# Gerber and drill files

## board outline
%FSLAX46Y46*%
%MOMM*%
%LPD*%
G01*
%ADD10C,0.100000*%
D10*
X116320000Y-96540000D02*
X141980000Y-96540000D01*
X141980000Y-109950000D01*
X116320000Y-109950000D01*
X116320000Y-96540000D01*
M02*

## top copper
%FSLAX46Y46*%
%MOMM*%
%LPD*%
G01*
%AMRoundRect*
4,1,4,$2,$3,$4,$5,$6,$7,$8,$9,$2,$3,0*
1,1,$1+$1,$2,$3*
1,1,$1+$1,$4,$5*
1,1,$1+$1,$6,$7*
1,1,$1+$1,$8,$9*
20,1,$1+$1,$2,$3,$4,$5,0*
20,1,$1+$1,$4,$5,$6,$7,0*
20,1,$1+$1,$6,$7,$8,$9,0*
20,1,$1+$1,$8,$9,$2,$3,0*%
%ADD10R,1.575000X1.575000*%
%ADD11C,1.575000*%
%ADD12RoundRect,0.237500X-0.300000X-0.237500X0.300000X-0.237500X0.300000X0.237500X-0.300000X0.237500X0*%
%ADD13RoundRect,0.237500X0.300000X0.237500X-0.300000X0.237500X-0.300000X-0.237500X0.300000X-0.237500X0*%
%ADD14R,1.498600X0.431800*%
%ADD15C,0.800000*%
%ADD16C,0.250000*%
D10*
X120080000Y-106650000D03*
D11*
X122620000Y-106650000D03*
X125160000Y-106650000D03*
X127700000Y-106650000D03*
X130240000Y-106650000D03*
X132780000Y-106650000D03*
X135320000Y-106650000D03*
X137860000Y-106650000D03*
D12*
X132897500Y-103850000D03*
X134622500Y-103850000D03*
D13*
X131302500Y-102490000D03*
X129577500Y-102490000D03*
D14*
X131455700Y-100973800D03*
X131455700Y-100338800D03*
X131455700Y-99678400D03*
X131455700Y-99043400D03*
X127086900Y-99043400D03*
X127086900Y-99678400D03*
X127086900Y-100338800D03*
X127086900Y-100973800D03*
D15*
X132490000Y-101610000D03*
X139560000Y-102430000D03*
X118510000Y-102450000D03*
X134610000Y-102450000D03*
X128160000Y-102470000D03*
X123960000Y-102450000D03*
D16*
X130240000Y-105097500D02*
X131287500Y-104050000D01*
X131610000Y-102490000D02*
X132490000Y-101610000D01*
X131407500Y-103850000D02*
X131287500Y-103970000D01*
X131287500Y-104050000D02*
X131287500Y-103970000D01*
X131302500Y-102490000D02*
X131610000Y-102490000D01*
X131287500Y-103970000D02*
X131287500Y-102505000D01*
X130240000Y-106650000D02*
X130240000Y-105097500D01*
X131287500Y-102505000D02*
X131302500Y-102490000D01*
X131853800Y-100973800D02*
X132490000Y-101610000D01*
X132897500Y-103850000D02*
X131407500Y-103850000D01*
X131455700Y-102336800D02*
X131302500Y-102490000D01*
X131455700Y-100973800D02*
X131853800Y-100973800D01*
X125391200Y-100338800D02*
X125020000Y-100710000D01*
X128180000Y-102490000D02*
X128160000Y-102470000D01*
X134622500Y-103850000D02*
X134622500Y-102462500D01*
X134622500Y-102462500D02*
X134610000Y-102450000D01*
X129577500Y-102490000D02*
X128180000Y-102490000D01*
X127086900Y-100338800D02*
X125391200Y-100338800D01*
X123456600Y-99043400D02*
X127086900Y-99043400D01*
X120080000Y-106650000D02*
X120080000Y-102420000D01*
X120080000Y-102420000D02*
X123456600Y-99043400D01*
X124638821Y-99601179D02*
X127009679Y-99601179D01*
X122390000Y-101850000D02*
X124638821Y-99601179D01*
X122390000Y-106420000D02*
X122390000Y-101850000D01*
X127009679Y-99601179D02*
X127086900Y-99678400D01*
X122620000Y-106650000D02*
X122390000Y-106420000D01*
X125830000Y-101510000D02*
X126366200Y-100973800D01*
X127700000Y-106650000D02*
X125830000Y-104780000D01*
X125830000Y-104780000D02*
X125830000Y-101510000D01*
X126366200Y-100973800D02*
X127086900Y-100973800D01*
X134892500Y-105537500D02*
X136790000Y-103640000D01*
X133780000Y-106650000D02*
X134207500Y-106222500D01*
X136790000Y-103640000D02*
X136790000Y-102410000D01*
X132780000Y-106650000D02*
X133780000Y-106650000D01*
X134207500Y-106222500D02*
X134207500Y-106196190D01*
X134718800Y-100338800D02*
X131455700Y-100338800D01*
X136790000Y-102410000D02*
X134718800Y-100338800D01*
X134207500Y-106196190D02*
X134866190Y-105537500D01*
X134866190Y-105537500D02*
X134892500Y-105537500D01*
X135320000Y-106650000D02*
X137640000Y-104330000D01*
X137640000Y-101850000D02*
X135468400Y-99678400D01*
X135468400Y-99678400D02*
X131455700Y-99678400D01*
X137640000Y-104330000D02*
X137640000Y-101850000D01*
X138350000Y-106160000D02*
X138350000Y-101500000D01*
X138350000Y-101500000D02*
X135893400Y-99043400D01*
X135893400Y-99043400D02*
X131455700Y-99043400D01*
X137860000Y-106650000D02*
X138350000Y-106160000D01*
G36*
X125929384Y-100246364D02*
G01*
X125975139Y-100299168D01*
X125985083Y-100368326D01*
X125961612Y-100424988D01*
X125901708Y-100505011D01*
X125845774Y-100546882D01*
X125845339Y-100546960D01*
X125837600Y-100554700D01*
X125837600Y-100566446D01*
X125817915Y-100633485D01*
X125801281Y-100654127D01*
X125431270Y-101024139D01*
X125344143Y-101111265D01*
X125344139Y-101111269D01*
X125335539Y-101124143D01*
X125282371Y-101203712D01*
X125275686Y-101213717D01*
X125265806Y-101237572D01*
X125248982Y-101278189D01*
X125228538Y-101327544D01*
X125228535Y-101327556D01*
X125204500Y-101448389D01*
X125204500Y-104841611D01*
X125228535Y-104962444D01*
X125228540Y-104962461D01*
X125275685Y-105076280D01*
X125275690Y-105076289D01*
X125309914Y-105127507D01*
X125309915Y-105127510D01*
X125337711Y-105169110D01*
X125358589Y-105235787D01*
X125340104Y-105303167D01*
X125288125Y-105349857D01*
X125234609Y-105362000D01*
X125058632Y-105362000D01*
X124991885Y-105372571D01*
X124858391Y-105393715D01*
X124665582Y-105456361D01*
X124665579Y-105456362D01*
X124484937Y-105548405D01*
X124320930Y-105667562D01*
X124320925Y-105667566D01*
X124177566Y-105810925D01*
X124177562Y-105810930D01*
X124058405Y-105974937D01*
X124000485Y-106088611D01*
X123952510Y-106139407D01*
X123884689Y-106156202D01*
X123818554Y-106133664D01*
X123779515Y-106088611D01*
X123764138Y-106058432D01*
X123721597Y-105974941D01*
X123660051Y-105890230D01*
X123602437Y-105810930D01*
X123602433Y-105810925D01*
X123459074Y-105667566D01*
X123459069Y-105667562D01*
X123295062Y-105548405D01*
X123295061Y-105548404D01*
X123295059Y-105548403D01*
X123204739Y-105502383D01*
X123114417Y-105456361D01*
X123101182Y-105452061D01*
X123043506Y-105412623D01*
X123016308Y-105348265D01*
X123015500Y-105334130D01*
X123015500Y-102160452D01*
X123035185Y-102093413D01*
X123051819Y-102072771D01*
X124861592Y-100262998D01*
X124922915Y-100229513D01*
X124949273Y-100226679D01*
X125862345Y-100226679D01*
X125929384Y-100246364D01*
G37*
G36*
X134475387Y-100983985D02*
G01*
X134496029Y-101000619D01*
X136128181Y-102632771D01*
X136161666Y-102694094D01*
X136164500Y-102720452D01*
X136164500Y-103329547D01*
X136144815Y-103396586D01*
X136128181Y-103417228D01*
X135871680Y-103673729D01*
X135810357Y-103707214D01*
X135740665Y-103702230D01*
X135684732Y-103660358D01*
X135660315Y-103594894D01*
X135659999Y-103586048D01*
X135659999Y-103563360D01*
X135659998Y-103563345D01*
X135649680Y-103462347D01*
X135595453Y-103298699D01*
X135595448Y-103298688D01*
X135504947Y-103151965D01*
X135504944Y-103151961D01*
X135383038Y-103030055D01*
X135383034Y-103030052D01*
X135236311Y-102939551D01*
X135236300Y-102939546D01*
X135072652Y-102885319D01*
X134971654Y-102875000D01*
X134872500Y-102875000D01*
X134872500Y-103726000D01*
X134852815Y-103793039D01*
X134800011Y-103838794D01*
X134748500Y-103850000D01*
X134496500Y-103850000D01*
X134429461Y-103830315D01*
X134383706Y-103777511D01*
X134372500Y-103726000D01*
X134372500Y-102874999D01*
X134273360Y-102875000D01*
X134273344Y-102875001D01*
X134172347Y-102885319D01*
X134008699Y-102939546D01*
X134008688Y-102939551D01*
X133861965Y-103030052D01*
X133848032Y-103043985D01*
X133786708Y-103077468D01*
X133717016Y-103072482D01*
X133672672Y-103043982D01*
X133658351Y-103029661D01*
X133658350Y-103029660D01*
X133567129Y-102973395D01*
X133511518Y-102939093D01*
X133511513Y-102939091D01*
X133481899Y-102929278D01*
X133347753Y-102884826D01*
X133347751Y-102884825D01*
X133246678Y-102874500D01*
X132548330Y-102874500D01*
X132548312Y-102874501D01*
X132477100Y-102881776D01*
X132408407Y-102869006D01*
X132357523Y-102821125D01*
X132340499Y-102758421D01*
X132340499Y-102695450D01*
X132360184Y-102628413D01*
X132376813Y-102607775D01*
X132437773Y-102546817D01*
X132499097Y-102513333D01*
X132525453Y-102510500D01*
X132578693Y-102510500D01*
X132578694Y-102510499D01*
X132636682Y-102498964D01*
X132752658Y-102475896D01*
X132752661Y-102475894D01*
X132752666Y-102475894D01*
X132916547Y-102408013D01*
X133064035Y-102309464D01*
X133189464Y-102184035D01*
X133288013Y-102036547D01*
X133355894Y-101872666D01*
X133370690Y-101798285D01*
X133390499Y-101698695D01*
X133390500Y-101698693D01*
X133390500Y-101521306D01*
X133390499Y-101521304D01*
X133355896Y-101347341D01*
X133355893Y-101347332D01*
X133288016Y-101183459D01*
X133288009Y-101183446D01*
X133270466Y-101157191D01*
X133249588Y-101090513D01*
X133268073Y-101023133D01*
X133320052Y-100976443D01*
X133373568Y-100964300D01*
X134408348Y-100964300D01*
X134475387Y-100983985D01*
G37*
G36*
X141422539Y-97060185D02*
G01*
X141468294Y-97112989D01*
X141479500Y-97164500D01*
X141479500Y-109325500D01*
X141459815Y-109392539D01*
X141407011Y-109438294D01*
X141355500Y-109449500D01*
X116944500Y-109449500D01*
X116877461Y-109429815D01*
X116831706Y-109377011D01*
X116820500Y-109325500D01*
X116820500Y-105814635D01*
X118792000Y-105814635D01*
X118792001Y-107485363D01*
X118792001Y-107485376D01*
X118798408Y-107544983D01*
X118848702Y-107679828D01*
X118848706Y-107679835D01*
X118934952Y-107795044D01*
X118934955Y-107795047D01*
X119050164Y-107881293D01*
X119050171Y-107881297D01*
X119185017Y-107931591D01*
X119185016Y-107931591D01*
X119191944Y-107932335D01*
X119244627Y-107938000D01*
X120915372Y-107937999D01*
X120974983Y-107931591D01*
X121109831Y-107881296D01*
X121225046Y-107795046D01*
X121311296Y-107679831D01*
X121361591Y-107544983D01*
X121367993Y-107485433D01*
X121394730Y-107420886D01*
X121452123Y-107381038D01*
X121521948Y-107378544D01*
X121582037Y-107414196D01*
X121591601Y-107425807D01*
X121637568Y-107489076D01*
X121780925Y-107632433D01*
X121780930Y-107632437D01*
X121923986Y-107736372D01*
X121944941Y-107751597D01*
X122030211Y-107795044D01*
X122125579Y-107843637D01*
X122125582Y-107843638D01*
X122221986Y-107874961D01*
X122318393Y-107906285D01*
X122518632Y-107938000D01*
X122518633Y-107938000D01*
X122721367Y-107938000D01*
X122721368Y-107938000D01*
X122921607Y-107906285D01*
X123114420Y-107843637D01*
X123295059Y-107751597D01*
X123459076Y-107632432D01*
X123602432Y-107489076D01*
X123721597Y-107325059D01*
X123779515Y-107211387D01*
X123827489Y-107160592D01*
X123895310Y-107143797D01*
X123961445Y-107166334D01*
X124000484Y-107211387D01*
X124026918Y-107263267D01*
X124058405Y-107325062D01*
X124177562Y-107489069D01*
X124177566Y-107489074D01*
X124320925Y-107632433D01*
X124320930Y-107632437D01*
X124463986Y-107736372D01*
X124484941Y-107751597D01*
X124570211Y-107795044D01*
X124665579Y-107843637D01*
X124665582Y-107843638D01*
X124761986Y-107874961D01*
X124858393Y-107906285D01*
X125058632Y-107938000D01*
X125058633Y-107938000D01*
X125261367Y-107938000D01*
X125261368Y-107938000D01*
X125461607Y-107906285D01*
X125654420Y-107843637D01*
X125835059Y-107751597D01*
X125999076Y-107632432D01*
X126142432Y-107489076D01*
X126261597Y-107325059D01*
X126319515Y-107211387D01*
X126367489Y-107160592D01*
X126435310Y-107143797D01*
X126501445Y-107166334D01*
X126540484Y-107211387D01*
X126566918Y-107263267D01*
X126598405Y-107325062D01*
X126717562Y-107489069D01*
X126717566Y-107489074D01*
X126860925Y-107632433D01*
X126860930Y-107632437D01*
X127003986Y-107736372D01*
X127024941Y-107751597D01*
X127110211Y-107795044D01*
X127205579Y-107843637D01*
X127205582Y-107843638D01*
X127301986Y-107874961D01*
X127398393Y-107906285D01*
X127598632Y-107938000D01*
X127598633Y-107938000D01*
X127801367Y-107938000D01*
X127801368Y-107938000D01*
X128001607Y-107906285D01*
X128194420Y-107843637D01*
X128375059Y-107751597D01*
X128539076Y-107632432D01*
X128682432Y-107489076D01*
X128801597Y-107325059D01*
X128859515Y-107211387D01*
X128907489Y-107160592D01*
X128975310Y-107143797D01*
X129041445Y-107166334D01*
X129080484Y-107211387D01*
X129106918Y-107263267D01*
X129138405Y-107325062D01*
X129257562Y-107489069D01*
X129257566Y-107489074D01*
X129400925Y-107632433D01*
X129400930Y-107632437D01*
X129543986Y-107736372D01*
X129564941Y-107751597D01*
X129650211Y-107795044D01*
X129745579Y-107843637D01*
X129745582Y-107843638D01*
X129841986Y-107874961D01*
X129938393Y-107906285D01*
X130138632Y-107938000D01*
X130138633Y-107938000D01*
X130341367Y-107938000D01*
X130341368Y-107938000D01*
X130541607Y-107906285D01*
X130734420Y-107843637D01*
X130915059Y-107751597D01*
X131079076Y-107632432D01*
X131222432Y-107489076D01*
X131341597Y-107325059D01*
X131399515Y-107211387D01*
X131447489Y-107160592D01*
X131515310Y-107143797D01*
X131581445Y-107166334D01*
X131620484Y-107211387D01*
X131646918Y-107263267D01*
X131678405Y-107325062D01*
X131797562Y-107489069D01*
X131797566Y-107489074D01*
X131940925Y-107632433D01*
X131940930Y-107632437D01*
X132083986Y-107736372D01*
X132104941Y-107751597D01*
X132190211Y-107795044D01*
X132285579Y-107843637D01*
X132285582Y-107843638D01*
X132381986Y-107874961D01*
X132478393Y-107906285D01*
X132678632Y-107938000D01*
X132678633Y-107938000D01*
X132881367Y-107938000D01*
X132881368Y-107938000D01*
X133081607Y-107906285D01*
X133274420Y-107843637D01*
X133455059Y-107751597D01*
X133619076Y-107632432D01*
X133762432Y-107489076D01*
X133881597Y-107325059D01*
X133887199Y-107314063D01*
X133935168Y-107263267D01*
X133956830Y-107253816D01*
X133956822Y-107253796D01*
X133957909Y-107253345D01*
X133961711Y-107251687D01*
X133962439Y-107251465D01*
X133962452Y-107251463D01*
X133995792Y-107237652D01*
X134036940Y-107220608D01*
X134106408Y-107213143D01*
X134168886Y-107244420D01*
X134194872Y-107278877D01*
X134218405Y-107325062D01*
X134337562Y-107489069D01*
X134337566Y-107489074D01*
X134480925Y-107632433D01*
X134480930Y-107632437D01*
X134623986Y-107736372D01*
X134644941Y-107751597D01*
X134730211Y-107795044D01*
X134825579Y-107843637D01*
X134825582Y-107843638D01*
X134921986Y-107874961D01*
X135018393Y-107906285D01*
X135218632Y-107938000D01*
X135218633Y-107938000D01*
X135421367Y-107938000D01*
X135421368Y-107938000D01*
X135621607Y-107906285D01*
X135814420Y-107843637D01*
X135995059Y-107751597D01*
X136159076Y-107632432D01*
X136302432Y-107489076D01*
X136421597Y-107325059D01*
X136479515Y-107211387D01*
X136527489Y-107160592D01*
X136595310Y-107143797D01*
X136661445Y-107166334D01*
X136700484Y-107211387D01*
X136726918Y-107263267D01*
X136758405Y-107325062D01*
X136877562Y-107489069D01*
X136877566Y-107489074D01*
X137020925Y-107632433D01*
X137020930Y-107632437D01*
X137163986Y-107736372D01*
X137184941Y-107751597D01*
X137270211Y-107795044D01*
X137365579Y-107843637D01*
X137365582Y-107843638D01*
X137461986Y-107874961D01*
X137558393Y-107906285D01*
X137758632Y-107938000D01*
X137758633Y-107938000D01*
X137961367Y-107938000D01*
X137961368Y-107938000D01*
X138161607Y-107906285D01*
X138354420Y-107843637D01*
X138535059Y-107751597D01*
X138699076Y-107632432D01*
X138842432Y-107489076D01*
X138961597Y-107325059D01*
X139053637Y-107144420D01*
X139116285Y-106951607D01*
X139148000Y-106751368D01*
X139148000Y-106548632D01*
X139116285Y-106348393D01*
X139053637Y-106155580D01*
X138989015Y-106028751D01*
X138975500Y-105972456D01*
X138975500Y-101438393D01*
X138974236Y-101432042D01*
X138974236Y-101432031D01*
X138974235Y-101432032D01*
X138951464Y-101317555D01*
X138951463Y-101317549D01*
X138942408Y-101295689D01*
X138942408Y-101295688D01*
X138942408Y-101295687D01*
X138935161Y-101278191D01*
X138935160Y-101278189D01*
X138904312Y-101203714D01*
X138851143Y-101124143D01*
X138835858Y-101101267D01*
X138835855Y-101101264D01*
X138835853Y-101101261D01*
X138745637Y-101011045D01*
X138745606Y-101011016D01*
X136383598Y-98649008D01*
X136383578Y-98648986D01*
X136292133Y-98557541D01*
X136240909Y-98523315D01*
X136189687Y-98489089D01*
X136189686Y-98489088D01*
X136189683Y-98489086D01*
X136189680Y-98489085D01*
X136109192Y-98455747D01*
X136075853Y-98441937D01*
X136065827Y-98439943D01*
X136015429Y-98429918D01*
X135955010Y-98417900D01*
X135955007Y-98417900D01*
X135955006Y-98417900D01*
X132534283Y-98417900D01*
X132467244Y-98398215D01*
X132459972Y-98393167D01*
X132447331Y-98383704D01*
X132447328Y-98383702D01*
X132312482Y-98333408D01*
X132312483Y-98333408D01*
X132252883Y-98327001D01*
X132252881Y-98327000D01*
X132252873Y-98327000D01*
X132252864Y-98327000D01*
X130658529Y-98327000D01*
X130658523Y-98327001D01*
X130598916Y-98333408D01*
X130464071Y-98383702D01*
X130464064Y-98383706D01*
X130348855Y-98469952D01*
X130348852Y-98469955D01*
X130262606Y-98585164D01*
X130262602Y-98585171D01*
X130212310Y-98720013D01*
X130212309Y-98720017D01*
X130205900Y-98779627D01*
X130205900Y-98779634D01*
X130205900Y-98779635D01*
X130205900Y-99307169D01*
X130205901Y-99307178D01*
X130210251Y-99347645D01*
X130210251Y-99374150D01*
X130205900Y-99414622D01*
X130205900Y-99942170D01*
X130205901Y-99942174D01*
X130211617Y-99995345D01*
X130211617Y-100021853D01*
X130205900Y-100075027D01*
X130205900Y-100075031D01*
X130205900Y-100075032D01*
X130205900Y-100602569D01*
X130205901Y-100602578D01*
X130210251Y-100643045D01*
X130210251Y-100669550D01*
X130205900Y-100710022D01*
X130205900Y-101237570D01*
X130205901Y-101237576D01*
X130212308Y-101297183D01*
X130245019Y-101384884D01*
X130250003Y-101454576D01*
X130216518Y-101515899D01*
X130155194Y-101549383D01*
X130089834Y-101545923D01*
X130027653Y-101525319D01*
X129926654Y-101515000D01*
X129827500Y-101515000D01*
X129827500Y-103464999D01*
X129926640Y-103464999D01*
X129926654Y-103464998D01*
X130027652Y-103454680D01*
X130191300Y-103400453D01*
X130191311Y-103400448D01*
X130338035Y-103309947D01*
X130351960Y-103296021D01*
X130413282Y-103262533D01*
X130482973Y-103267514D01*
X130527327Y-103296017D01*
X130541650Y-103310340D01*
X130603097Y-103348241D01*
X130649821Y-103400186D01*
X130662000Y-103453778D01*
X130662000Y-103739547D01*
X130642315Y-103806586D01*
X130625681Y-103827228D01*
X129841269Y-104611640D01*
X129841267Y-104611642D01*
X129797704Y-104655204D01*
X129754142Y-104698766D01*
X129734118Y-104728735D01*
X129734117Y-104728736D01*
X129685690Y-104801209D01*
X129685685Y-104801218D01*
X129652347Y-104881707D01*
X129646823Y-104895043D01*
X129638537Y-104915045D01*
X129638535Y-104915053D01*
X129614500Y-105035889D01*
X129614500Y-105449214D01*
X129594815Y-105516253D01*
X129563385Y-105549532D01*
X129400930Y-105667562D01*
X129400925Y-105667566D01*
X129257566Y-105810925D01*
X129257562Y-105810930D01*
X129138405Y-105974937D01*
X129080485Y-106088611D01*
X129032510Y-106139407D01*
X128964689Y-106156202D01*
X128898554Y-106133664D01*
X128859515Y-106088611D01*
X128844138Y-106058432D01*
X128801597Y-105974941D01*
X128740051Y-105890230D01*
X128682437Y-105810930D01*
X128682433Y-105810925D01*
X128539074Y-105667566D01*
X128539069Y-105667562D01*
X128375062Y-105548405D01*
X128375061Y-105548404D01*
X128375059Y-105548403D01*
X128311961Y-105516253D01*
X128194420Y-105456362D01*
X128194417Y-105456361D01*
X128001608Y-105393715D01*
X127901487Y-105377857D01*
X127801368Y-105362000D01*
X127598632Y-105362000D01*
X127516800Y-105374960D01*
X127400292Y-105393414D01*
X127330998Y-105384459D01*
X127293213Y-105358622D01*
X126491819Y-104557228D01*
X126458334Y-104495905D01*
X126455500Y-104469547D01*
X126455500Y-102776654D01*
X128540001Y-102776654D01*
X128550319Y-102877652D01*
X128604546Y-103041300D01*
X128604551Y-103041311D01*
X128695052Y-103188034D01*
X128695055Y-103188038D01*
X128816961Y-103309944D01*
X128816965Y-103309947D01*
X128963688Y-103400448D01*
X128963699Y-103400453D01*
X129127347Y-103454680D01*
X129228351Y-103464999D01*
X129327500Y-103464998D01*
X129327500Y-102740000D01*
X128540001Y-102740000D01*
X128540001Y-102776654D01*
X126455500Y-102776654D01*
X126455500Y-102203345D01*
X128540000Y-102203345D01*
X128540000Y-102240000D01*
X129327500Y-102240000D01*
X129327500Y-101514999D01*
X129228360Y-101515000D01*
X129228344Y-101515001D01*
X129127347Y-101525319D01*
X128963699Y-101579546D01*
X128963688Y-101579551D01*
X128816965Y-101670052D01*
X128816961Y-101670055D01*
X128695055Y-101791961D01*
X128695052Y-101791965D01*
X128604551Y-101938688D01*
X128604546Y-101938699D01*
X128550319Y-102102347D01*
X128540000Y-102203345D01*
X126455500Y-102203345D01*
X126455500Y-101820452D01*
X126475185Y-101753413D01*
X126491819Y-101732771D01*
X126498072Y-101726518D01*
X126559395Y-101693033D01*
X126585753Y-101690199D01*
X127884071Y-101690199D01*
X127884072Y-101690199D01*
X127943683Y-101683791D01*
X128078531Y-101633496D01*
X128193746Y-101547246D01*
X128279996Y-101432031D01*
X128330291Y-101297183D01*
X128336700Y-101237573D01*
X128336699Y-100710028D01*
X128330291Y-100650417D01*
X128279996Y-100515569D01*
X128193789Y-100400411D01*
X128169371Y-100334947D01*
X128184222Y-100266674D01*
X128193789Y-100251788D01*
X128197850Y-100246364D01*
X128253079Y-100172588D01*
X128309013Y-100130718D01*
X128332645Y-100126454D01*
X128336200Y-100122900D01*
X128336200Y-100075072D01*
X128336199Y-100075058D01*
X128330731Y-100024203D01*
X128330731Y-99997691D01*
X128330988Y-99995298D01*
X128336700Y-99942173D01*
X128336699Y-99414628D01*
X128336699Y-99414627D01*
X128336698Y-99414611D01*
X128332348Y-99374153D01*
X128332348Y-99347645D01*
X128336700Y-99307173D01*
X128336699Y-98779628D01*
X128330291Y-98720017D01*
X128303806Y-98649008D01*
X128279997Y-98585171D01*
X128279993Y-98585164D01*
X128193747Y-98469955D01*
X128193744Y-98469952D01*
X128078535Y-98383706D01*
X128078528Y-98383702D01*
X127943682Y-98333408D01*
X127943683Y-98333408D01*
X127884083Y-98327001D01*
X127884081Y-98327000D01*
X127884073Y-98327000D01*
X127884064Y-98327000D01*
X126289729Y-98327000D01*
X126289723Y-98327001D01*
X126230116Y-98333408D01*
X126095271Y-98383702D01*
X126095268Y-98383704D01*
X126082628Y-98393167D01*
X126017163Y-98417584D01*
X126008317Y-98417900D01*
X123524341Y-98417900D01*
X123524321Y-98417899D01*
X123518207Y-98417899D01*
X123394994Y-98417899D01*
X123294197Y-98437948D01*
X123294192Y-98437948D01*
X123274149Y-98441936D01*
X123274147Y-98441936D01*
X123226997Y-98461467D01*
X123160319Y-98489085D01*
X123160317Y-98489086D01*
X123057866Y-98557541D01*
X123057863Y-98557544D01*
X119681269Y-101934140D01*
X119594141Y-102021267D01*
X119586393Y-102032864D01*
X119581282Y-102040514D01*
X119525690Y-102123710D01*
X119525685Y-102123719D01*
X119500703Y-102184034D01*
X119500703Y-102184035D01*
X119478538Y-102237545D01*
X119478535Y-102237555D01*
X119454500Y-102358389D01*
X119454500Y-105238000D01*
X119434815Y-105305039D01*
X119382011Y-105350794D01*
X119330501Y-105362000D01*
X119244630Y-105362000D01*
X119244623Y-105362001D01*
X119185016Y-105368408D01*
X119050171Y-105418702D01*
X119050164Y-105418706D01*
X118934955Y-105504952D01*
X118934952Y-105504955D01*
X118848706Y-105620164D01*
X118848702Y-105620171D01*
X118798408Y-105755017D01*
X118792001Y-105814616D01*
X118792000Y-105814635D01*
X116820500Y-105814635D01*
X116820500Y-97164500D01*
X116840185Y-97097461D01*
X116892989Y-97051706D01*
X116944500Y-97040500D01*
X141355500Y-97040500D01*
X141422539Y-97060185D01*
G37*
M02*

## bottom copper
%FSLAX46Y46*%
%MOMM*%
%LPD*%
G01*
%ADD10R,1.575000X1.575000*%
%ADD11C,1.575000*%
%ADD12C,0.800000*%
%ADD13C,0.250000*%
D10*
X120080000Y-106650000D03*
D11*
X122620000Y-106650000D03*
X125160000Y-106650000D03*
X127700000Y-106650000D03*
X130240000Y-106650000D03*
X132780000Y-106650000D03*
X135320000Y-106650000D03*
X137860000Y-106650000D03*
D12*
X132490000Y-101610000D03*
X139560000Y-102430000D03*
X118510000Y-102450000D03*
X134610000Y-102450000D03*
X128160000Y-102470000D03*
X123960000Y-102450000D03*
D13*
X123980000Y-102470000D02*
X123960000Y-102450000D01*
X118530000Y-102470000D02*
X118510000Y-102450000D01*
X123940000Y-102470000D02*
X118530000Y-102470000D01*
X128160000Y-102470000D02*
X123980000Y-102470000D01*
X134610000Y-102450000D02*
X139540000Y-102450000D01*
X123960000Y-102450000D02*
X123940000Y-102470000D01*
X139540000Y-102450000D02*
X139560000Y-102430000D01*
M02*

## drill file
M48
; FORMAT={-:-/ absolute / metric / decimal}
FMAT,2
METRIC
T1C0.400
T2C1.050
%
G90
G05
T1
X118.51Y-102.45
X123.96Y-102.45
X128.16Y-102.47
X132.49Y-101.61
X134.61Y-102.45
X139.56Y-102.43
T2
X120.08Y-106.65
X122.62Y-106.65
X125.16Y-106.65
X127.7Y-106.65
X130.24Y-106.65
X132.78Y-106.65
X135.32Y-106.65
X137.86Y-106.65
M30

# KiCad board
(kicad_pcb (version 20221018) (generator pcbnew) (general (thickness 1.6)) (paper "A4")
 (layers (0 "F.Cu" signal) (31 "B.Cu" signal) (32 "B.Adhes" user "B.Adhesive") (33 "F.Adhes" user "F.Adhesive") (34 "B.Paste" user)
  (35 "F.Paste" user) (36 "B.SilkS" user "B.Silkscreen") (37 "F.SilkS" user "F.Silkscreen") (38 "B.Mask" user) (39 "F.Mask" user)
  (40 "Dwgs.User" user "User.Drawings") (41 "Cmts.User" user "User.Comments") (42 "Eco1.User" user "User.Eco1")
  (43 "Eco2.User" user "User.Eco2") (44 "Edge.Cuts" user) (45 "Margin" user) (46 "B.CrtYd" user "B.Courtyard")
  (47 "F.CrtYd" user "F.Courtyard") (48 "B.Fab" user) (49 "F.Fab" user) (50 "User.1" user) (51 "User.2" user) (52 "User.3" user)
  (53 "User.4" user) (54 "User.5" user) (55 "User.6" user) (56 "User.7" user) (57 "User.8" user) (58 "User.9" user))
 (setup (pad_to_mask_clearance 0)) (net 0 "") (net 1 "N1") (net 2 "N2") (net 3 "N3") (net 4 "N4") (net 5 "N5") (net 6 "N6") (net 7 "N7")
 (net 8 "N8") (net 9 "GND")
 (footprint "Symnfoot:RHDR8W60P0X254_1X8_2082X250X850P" (layer "F.Cu") (at 120.08 106.65)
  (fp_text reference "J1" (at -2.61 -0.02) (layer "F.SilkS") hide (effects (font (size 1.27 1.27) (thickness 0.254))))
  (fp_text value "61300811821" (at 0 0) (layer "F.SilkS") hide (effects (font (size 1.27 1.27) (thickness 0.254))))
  (pad "1" thru_hole rect (at 0 0) (size 1.575 1.575) (drill 1.05) (layers "*.Cu" "*.Mask") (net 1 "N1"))
  (pad "2" thru_hole circle (at 2.54 0) (size 1.575 1.575) (drill 1.05) (layers "*.Cu" "*.Mask") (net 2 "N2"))
  (pad "3" thru_hole circle (at 5.08 0) (size 1.575 1.575) (drill 1.05) (layers "*.Cu" "*.Mask") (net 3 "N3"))
  (pad "4" thru_hole circle (at 7.62 0) (size 1.575 1.575) (drill 1.05) (layers "*.Cu" "*.Mask") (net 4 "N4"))
  (pad "5" thru_hole circle (at 10.16 0) (size 1.575 1.575) (drill 1.05) (layers "*.Cu" "*.Mask") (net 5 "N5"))
  (pad "6" thru_hole circle (at 12.7 0) (size 1.575 1.575) (drill 1.05) (layers "*.Cu" "*.Mask") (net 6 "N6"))
  (pad "7" thru_hole circle (at 15.24 0) (size 1.575 1.575) (drill 1.05) (layers "*.Cu" "*.Mask") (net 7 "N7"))
  (pad "8" thru_hole circle (at 17.78 0) (size 1.575 1.575) (drill 1.05) (layers "*.Cu" "*.Mask") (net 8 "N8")))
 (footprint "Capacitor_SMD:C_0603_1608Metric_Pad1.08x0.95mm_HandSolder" (layer "F.Cu") (at 133.76 103.85)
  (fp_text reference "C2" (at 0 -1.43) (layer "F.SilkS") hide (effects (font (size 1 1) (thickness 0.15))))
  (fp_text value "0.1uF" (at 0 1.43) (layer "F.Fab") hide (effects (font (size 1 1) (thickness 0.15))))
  (pad "1" smd roundrect (at -0.8625 0) (size 1.075 0.95) (layers "F.Cu" "F.Paste" "F.Mask") (roundrect_rratio 0.25) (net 5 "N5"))
  (pad "2" smd roundrect (at 0.8625 0) (size 1.075 0.95) (layers "F.Cu" "F.Paste" "F.Mask") (roundrect_rratio 0.25) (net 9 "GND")))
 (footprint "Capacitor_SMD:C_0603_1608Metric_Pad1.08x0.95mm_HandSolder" (layer "F.Cu") (at 130.44 102.49 180)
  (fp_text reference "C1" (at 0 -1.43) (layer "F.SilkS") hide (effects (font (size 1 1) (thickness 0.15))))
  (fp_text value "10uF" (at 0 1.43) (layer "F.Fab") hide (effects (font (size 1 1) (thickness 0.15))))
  (pad "1" smd roundrect (at -0.8625 0 180) (size 1.075 0.95) (layers "F.Cu" "F.Paste" "F.Mask") (roundrect_rratio 0.25) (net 5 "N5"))
  (pad "2" smd roundrect (at 0.8625 0 180) (size 1.075 0.95) (layers "F.Cu" "F.Paste" "F.Mask") (roundrect_rratio 0.25) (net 9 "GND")))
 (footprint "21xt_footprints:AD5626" (layer "F.Cu") (at 129.2713 100.0086 180)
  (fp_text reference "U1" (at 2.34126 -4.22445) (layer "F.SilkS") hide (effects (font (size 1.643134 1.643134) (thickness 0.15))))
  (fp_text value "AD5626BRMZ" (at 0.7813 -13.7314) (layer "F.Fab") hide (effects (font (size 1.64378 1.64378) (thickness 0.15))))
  (pad "1" smd rect (at -2.1844 -0.9652 180) (size 1.4986 0.4318) (layers "F.Cu" "F.Paste" "F.Mask") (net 5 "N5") (solder_mask_margin 0.102))
  (pad "2" smd rect (at -2.1844 -0.3302 180) (size 1.4986 0.4318) (layers "F.Cu" "F.Paste" "F.Mask") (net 6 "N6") (solder_mask_margin 0.102))
  (pad "3" smd rect (at -2.1844 0.3302 180) (size 1.4986 0.4318) (layers "F.Cu" "F.Paste" "F.Mask") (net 7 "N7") (solder_mask_margin 0.102))
  (pad "4" smd rect (at -2.1844 0.9652 180) (size 1.4986 0.4318) (layers "F.Cu" "F.Paste" "F.Mask") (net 8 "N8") (solder_mask_margin 0.102))
  (pad "5" smd rect (at 2.1844 0.9652 180) (size 1.4986 0.4318) (layers "F.Cu" "F.Paste" "F.Mask") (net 1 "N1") (solder_mask_margin 0.102))
  (pad "6" smd rect (at 2.1844 0.3302 180) (size 1.4986 0.4318) (layers "F.Cu" "F.Paste" "F.Mask") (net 2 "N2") (solder_mask_margin 0.102))
  (pad "7" smd rect (at 2.1844 -0.3302 180) (size 1.4986 0.4318) (layers "F.Cu" "F.Paste" "F.Mask") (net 9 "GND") (solder_mask_margin 0.102))
  (pad "8" smd rect (at 2.1844 -0.9652 180) (size 1.4986 0.4318) (layers "F.Cu" "F.Paste" "F.Mask") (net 4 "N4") (solder_mask_margin 0.102)))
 (gr_rect (start 116.32 96.54) (end 141.98 109.95) (stroke (width 0.1) (type default)) (fill none) (layer "Edge.Cuts"))
 (segment (start 130.24 105.0975) (end 131.2875 104.05) (width 0.25) (layer "F.Cu") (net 5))
 (segment (start 131.61 102.49) (end 132.49 101.61) (width 0.25) (layer "F.Cu") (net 5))
 (segment (start 131.4075 103.85) (end 131.2875 103.97) (width 0.25) (layer "F.Cu") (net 5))
 (segment (start 131.2875 104.05) (end 131.2875 103.97) (width 0.25) (layer "F.Cu") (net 5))
 (segment (start 131.3025 102.49) (end 131.61 102.49) (width 0.25) (layer "F.Cu") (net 5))
 (segment (start 131.2875 103.97) (end 131.2875 102.505) (width 0.25) (layer "F.Cu") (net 5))
 (segment (start 130.24 106.65) (end 130.24 105.0975) (width 0.25) (layer "F.Cu") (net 5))
 (segment (start 131.2875 102.505) (end 131.3025 102.49) (width 0.25) (layer "F.Cu") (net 5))
 (segment (start 131.8538 100.9738) (end 132.49 101.61) (width 0.25) (layer "F.Cu") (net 5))
 (segment (start 132.8975 103.85) (end 131.4075 103.85) (width 0.25) (layer "F.Cu") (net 5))
 (segment (start 131.4557 102.3368) (end 131.3025 102.49) (width 0.25) (layer "F.Cu") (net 5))
 (segment (start 131.4557 100.9738) (end 131.8538 100.9738) (width 0.25) (layer "F.Cu") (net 5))
 (via (at 132.49 101.61) (size 0.8) (drill 0.4) (layers "F.Cu" "B.Cu") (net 5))
 (segment (start 125.3912 100.3388) (end 125.02 100.71) (width 0.25) (layer "F.Cu") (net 9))
 (segment (start 128.18 102.49) (end 128.16 102.47) (width 0.25) (layer "F.Cu") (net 9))
 (segment (start 134.6225 103.85) (end 134.6225 102.4625) (width 0.25) (layer "F.Cu") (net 9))
 (segment (start 134.6225 102.4625) (end 134.61 102.45) (width 0.25) (layer "F.Cu") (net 9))
 (segment (start 129.5775 102.49) (end 128.18 102.49) (width 0.25) (layer "F.Cu") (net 9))
 (segment (start 127.0869 100.3388) (end 125.3912 100.3388) (width 0.25) (layer "F.Cu") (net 9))
 (via (at 139.56 102.43) (size 0.8) (drill 0.4) (layers "F.Cu" "B.Cu") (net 9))
 (via (at 118.51 102.45) (size 0.8) (drill 0.4) (layers "F.Cu" "B.Cu") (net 9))
 (via (at 134.61 102.45) (size 0.8) (drill 0.4) (layers "F.Cu" "B.Cu") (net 9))
 (via (at 128.16 102.47) (size 0.8) (drill 0.4) (layers "F.Cu" "B.Cu") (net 9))
 (via (at 123.96 102.45) (size 0.8) (drill 0.4) (layers "F.Cu" "B.Cu") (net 9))
 (segment (start 123.98 102.47) (end 123.96 102.45) (width 0.25) (layer "B.Cu") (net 9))
 (segment (start 118.53 102.47) (end 118.51 102.45) (width 0.25) (layer "B.Cu") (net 9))
 (segment (start 123.94 102.47) (end 118.53 102.47) (width 0.25) (layer "B.Cu") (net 9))
 (segment (start 128.16 102.47) (end 123.98 102.47) (width 0.25) (layer "B.Cu") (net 9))
 (segment (start 134.61 102.45) (end 139.54 102.45) (width 0.25) (layer "B.Cu") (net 9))
 (segment (start 123.96 102.45) (end 123.94 102.47) (width 0.25) (layer "B.Cu") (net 9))
 (segment (start 139.54 102.45) (end 139.56 102.43) (width 0.25) (layer "B.Cu") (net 9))
 (segment (start 123.4566 99.0434) (end 127.0869 99.0434) (width 0.25) (layer "F.Cu") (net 1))
 (segment (start 120.08 106.65) (end 120.08 102.42) (width 0.25) (layer "F.Cu") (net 1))
 (segment (start 120.08 102.42) (end 123.4566 99.0434) (width 0.25) (layer "F.Cu") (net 1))
 (segment (start 124.638821 99.601179) (end 127.009679 99.601179) (width 0.25) (layer "F.Cu") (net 2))
 (segment (start 122.39 101.85) (end 124.638821 99.601179) (width 0.25) (layer "F.Cu") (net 2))
 (segment (start 122.39 106.42) (end 122.39 101.85) (width 0.25) (layer "F.Cu") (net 2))
 (segment (start 127.009679 99.601179) (end 127.0869 99.6784) (width 0.25) (layer "F.Cu") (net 2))
 (segment (start 122.62 106.65) (end 122.39 106.42) (width 0.25) (layer "F.Cu") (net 2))
 (segment (start 125.83 101.51) (end 126.3662 100.9738) (width 0.25) (layer "F.Cu") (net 4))
 (segment (start 127.7 106.65) (end 125.83 104.78) (width 0.25) (layer "F.Cu") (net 4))
 (segment (start 125.83 104.78) (end 125.83 101.51) (width 0.25) (layer "F.Cu") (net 4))
 (segment (start 126.3662 100.9738) (end 127.0869 100.9738) (width 0.25) (layer "F.Cu") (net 4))
 (segment (start 134.8925 105.5375) (end 136.79 103.64) (width 0.25) (layer "F.Cu") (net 6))
 (segment (start 133.78 106.65) (end 134.2075 106.2225) (width 0.25) (layer "F.Cu") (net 6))
 (segment (start 136.79 103.64) (end 136.79 102.41) (width 0.25) (layer "F.Cu") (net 6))
 (segment (start 132.78 106.65) (end 133.78 106.65) (width 0.25) (layer "F.Cu") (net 6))
 (segment (start 134.2075 106.2225) (end 134.2075 106.19619) (width 0.25) (layer "F.Cu") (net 6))
 (segment (start 134.7188 100.3388) (end 131.4557 100.3388) (width 0.25) (layer "F.Cu") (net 6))
 (segment (start 136.79 102.41) (end 134.7188 100.3388) (width 0.25) (layer "F.Cu") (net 6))
 (segment (start 134.2075 106.19619) (end 134.86619 105.5375) (width 0.25) (layer "F.Cu") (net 6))
 (segment (start 134.86619 105.5375) (end 134.8925 105.5375) (width 0.25) (layer "F.Cu") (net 6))
 (segment (start 135.32 106.65) (end 137.64 104.33) (width 0.25) (layer "F.Cu") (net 7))
 (segment (start 137.64 101.85) (end 135.4684 99.6784) (width 0.25) (layer "F.Cu") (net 7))
 (segment (start 135.4684 99.6784) (end 131.4557 99.6784) (width 0.25) (layer "F.Cu") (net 7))
 (segment (start 137.64 104.33) (end 137.64 101.85) (width 0.25) (layer "F.Cu") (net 7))
 (segment (start 138.35 106.16) (end 138.35 101.5) (width 0.25) (layer "F.Cu") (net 8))
 (segment (start 138.35 101.5) (end 135.8934 99.0434) (width 0.25) (layer "F.Cu") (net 8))
 (segment (start 135.8934 99.0434) (end 131.4557 99.0434) (width 0.25) (layer "F.Cu") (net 8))
 (segment (start 137.86 106.65) (end 138.35 106.16) (width 0.25) (layer "F.Cu") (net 8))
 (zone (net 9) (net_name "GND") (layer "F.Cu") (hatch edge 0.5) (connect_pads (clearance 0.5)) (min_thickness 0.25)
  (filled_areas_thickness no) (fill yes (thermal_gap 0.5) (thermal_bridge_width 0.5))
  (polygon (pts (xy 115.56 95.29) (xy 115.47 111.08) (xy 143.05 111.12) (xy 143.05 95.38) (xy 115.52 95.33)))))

